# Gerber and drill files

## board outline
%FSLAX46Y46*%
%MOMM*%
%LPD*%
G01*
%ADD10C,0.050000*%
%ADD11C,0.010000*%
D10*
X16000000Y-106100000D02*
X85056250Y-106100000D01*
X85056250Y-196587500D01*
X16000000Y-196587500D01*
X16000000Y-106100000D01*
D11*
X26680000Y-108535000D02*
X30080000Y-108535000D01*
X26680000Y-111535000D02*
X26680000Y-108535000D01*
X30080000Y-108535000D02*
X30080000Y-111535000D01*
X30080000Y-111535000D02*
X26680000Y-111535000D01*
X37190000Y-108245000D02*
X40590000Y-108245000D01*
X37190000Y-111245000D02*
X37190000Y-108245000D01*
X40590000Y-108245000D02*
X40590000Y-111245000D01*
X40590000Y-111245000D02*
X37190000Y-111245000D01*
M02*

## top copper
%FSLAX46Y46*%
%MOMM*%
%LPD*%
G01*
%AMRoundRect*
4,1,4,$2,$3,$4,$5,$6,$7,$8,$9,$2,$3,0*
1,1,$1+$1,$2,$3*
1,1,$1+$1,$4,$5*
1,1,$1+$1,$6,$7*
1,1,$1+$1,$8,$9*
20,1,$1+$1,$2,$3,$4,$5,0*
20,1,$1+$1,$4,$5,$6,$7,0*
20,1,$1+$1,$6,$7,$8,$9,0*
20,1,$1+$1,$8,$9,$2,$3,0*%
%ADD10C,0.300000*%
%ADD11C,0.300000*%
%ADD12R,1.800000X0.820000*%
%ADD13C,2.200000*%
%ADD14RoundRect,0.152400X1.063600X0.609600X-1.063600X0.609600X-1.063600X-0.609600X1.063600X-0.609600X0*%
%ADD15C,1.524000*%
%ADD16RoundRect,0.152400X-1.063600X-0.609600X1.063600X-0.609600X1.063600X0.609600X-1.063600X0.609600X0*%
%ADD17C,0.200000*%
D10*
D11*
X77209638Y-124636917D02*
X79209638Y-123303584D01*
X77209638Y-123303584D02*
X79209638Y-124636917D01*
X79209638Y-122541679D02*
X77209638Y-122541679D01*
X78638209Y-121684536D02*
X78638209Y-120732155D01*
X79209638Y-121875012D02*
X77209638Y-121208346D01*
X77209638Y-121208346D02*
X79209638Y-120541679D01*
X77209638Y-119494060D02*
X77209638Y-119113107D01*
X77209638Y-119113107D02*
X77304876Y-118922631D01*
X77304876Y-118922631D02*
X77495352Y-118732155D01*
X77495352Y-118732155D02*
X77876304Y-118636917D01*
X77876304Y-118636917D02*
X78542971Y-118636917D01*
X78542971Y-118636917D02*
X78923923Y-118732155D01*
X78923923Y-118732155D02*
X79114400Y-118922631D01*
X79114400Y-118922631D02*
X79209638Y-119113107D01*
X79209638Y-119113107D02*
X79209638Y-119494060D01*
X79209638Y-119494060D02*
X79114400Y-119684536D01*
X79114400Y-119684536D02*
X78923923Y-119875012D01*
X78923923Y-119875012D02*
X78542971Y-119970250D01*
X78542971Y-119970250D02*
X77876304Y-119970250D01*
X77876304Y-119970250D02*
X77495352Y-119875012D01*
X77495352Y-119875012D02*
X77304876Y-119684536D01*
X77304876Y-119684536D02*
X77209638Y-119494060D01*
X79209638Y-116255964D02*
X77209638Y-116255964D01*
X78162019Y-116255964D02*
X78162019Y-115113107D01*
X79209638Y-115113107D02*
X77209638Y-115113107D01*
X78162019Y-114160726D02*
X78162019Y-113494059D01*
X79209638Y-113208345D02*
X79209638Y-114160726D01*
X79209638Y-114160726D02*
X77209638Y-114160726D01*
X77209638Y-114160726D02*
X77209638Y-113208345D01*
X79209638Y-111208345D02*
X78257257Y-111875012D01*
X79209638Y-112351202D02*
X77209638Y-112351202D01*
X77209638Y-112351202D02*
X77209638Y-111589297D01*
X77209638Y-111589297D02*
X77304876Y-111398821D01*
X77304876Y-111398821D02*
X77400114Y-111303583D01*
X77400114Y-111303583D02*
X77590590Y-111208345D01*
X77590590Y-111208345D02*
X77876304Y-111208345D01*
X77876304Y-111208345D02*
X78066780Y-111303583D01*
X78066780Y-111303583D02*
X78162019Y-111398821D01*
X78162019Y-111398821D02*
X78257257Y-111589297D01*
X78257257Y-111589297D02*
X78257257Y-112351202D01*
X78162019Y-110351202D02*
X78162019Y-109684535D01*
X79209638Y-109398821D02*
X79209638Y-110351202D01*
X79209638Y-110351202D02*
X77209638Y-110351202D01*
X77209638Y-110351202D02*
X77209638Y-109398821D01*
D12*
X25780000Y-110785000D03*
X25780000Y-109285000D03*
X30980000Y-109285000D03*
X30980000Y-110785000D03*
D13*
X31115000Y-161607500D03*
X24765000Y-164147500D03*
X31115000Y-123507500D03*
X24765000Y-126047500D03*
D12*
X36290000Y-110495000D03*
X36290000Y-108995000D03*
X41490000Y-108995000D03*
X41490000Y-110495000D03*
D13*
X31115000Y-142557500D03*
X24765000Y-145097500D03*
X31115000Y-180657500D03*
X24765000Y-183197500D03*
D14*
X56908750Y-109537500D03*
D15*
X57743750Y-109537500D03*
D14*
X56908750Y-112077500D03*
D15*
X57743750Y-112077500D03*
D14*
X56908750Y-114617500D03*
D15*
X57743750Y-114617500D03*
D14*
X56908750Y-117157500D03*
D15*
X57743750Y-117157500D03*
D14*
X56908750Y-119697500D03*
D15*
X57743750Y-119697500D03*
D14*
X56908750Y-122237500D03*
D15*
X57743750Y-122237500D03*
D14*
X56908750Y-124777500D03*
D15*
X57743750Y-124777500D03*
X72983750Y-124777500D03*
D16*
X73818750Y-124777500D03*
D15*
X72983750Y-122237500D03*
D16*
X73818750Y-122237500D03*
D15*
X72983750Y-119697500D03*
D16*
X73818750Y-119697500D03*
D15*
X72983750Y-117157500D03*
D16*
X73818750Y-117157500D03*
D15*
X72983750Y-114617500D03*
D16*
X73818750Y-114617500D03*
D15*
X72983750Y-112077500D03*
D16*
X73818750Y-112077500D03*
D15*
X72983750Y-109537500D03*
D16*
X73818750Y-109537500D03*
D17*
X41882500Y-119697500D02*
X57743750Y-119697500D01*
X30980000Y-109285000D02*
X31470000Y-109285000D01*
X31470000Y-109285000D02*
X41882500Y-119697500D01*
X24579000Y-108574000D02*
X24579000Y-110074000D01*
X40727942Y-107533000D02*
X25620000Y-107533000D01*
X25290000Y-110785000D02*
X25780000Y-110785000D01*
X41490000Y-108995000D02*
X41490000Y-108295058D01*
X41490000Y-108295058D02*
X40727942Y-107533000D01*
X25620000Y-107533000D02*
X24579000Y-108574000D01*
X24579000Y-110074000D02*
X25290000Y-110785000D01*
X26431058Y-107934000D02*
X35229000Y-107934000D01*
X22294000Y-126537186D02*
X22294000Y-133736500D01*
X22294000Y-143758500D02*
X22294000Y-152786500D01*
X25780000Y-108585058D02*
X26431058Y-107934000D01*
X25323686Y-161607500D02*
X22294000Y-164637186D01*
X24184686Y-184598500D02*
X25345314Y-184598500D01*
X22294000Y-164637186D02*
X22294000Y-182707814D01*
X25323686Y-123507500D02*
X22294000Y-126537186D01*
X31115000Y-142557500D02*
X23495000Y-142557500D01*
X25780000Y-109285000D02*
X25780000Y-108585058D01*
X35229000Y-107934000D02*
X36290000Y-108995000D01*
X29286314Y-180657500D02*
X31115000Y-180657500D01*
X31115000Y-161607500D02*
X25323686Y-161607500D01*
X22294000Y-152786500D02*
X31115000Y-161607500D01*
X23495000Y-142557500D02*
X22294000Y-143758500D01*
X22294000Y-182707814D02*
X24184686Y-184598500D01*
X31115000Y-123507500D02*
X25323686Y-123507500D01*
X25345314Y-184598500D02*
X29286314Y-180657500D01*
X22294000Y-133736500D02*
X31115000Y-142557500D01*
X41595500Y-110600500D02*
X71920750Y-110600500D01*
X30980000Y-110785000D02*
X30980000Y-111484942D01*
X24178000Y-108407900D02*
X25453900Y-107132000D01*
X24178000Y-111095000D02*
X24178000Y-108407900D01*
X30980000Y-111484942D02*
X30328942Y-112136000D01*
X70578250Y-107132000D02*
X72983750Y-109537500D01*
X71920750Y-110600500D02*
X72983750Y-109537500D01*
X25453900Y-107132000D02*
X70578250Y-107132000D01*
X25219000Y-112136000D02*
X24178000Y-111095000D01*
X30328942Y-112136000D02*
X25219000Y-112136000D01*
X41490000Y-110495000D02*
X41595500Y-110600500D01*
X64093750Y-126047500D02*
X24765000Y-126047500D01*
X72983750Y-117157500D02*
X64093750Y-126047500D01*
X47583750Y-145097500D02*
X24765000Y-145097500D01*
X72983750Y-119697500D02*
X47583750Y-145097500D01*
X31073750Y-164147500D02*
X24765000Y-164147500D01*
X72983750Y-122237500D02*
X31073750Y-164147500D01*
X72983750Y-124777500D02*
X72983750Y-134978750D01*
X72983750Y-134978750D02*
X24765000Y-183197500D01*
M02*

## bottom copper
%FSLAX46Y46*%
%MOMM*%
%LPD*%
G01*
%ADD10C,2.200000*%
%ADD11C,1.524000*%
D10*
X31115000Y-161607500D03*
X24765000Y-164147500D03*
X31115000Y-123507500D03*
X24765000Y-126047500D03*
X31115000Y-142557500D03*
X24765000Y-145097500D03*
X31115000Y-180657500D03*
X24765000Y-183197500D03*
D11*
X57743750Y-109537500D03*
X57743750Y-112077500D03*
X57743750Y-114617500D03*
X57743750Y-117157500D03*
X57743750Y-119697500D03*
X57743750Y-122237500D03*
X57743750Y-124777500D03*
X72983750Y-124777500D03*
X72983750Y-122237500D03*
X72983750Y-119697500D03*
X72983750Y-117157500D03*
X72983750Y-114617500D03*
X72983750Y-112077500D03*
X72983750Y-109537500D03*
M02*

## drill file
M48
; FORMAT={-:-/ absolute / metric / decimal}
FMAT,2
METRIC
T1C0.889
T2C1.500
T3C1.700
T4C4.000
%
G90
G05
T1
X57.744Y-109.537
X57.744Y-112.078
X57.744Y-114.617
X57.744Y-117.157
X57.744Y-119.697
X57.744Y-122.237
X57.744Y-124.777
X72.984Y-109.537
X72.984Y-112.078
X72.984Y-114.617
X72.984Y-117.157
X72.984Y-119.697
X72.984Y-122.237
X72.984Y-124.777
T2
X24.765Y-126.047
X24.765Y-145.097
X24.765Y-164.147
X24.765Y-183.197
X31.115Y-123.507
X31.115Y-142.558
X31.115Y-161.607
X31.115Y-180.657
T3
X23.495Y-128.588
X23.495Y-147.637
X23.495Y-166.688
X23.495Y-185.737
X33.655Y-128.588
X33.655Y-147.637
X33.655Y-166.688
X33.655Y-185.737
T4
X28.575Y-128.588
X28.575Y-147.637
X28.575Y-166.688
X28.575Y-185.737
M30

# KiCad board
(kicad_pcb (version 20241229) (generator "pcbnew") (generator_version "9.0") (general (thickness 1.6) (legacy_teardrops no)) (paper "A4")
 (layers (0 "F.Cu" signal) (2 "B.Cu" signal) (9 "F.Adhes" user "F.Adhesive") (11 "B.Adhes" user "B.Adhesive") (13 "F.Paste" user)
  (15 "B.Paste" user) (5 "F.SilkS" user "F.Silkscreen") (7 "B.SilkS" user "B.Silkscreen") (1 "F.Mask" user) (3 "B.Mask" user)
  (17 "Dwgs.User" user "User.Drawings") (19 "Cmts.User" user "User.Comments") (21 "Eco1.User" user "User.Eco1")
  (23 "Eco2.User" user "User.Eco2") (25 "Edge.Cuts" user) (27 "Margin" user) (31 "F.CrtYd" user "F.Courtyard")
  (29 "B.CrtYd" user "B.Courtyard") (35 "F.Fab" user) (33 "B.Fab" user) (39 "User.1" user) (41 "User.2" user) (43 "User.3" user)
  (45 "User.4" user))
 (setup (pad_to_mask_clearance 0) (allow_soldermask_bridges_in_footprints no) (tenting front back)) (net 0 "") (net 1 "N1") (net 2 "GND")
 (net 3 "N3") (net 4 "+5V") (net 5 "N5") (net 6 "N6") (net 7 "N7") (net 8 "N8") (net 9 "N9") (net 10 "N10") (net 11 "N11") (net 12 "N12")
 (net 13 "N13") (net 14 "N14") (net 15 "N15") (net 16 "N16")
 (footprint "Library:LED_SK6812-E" (layer "F.Cu") (at 28.38 110.035 180)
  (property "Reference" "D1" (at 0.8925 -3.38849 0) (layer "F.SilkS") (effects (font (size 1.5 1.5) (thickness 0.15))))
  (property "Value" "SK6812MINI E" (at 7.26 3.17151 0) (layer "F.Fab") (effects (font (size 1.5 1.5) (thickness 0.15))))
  (fp_line (start 1.7 1.5) (end -1.7 1.5) (stroke (width 0.01) (type solid)) (layer "Edge.Cuts"))
  (fp_line (start 1.7 -1.5) (end 1.7 1.5) (stroke (width 0.01) (type solid)) (layer "Edge.Cuts"))
  (fp_line (start -1.7 1.5) (end -1.7 -1.5) (stroke (width 0.01) (type solid)) (layer "Edge.Cuts"))
  (fp_line (start -1.7 -1.5) (end 1.7 -1.5) (stroke (width 0.01) (type solid)) (layer "Edge.Cuts"))
  (pad "1" smd rect (at 2.6 -0.75 180) (size 1.8 0.82) (layers "F.Cu" "F.Mask" "F.Paste") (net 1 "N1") (solder_mask_margin 0.102))
  (pad "2" smd rect (at 2.6 0.75 180) (size 1.8 0.82) (layers "F.Cu" "F.Mask" "F.Paste") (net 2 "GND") (solder_mask_margin 0.102))
  (pad "3" smd rect (at -2.6 0.75 180) (size 1.8 0.82) (layers "F.Cu" "F.Mask" "F.Paste") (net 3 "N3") (solder_mask_margin 0.102))
  (pad "4" smd rect (at -2.6 -0.75 180) (size 1.8 0.82) (layers "F.Cu" "F.Mask" "F.Paste") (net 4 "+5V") (solder_mask_margin 0.102)))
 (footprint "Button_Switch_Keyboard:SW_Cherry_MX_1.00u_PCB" (layer "F.Cu") (at 31.115 161.6075)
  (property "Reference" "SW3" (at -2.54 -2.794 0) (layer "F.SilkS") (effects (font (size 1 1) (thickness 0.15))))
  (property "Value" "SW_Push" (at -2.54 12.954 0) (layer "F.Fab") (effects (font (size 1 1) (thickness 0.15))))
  (pad "" np_thru_hole circle (at -7.62 5.08) (size 1.7 1.7) (drill 1.7) (layers "*.Cu" "*.Mask"))
  (pad "" np_thru_hole circle (at -2.54 5.08) (size 4 4) (drill 4) (layers "*.Cu" "*.Mask"))
  (pad "" np_thru_hole circle (at 2.54 5.08) (size 1.7 1.7) (drill 1.7) (layers "*.Cu" "*.Mask"))
  (pad "1" thru_hole circle (at 0 0) (size 2.2 2.2) (drill 1.5) (layers "*.Cu" "*.Mask") (remove_unused_layers no) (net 2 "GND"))
  (pad "2" thru_hole circle (at -6.35 2.54) (size 2.2 2.2) (drill 1.5) (layers "*.Cu" "*.Mask") (remove_unused_layers no) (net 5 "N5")))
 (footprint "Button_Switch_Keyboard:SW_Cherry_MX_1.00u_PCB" (layer "F.Cu") (at 31.115 123.5075)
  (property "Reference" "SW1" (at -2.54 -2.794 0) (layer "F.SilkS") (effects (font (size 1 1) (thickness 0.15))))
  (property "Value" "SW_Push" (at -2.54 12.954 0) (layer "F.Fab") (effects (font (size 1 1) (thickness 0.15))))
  (pad "" np_thru_hole circle (at -7.62 5.08) (size 1.7 1.7) (drill 1.7) (layers "*.Cu" "*.Mask"))
  (pad "" np_thru_hole circle (at -2.54 5.08) (size 4 4) (drill 4) (layers "*.Cu" "*.Mask"))
  (pad "" np_thru_hole circle (at 2.54 5.08) (size 1.7 1.7) (drill 1.7) (layers "*.Cu" "*.Mask"))
  (pad "1" thru_hole circle (at 0 0) (size 2.2 2.2) (drill 1.5) (layers "*.Cu" "*.Mask") (remove_unused_layers no) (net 2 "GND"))
  (pad "2" thru_hole circle (at -6.35 2.54) (size 2.2 2.2) (drill 1.5) (layers "*.Cu" "*.Mask") (remove_unused_layers no) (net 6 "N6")))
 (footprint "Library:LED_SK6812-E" (layer "F.Cu") (at 38.89 109.745 180)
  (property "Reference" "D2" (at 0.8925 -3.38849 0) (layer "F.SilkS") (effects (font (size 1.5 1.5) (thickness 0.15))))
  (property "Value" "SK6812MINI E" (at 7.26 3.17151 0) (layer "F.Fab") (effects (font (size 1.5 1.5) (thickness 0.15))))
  (fp_line (start 1.7 1.5) (end -1.7 1.5) (stroke (width 0.01) (type solid)) (layer "Edge.Cuts"))
  (fp_line (start 1.7 -1.5) (end 1.7 1.5) (stroke (width 0.01) (type solid)) (layer "Edge.Cuts"))
  (fp_line (start -1.7 1.5) (end -1.7 -1.5) (stroke (width 0.01) (type solid)) (layer "Edge.Cuts"))
  (fp_line (start -1.7 -1.5) (end 1.7 -1.5) (stroke (width 0.01) (type solid)) (layer "Edge.Cuts"))
  (pad "1" smd rect (at 2.6 -0.75 180) (size 1.8 0.82) (layers "F.Cu" "F.Mask" "F.Paste") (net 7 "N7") (solder_mask_margin 0.102))
  (pad "2" smd rect (at 2.6 0.75 180) (size 1.8 0.82) (layers "F.Cu" "F.Mask" "F.Paste") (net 2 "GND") (solder_mask_margin 0.102))
  (pad "3" smd rect (at -2.6 0.75 180) (size 1.8 0.82) (layers "F.Cu" "F.Mask" "F.Paste") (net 1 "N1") (solder_mask_margin 0.102))
  (pad "4" smd rect (at -2.6 -0.75 180) (size 1.8 0.82) (layers "F.Cu" "F.Mask" "F.Paste") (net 4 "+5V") (solder_mask_margin 0.102)))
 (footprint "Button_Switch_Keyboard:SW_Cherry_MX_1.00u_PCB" (layer "F.Cu") (at 31.115 142.5575)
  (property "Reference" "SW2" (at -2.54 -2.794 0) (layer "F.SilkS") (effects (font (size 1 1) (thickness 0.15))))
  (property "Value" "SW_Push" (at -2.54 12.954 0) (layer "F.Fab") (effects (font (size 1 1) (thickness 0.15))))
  (pad "" np_thru_hole circle (at -7.62 5.08) (size 1.7 1.7) (drill 1.7) (layers "*.Cu" "*.Mask"))
  (pad "" np_thru_hole circle (at -2.54 5.08) (size 4 4) (drill 4) (layers "*.Cu" "*.Mask"))
  (pad "" np_thru_hole circle (at 2.54 5.08) (size 1.7 1.7) (drill 1.7) (layers "*.Cu" "*.Mask"))
  (pad "1" thru_hole circle (at 0 0) (size 2.2 2.2) (drill 1.5) (layers "*.Cu" "*.Mask") (remove_unused_layers no) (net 2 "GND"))
  (pad "2" thru_hole circle (at -6.35 2.54) (size 2.2 2.2) (drill 1.5) (layers "*.Cu" "*.Mask") (remove_unused_layers no) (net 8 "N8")))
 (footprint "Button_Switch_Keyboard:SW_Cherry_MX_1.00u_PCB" (layer "F.Cu") (at 31.115 180.6575)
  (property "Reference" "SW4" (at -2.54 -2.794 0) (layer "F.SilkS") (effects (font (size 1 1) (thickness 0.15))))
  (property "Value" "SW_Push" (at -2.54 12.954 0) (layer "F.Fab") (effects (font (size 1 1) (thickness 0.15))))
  (pad "" np_thru_hole circle (at -7.62 5.08) (size 1.7 1.7) (drill 1.7) (layers "*.Cu" "*.Mask"))
  (pad "" np_thru_hole circle (at -2.54 5.08) (size 4 4) (drill 4) (layers "*.Cu" "*.Mask"))
  (pad "" np_thru_hole circle (at 2.54 5.08) (size 1.7 1.7) (drill 1.7) (layers "*.Cu" "*.Mask"))
  (pad "1" thru_hole circle (at 0 0) (size 2.2 2.2) (drill 1.5) (layers "*.Cu" "*.Mask") (remove_unused_layers no) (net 2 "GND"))
  (pad "2" thru_hole circle (at -6.35 2.54) (size 2.2 2.2) (drill 1.5) (layers "*.Cu" "*.Mask") (remove_unused_layers no) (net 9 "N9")))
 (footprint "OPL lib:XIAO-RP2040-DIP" (layer "F.Cu") (at 65.36375 117.1575)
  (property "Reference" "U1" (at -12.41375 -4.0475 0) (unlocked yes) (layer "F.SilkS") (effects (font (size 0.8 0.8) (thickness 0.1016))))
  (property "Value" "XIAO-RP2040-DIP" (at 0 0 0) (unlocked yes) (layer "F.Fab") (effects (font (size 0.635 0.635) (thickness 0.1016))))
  (pad "1" smd roundrect (at -8.455 -7.62 180) (size 2.432 1.524) (layers "F.Cu" "F.Mask") (roundrect_rratio 0.1) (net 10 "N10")
   (thermal_bridge_angle 45))
  (pad "1" thru_hole circle (at -7.62 -7.62 180) (size 1.524 1.524) (drill 0.889) (layers "*.Cu" "*.Mask") (remove_unused_layers no)
   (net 10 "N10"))
  (pad "2" smd roundrect (at -8.455 -5.08 180) (size 2.432 1.524) (layers "F.Cu" "F.Mask") (roundrect_rratio 0.1) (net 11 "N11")
   (thermal_bridge_angle 45))
  (pad "2" thru_hole circle (at -7.62 -5.08 180) (size 1.524 1.524) (drill 0.889) (layers "*.Cu" "*.Mask") (remove_unused_layers no)
   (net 11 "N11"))
  (pad "3" smd roundrect (at -8.455 -2.54 180) (size 2.432 1.524) (layers "F.Cu" "F.Mask") (roundrect_rratio 0.1) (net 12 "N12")
   (thermal_bridge_angle 45))
  (pad "3" thru_hole circle (at -7.62 -2.54 180) (size 1.524 1.524) (drill 0.889) (layers "*.Cu" "*.Mask") (remove_unused_layers no)
   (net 12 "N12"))
  (pad "4" smd roundrect (at -8.455 0 180) (size 2.432 1.524) (layers "F.Cu" "F.Mask") (roundrect_rratio 0.1) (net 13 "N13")
   (thermal_bridge_angle 45))
  (pad "4" thru_hole circle (at -7.62 0 180) (size 1.524 1.524) (drill 0.889) (layers "*.Cu" "*.Mask") (remove_unused_layers no)
   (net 13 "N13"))
  (pad "5" smd roundrect (at -8.455 2.54 180) (size 2.432 1.524) (layers "F.Cu" "F.Mask") (roundrect_rratio 0.1) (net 3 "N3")
   (thermal_bridge_angle 45))
  (pad "5" thru_hole circle (at -7.62 2.54 180) (size 1.524 1.524) (drill 0.889) (layers "*.Cu" "*.Mask") (remove_unused_layers no)
   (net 3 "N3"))
  (pad "6" smd roundrect (at -8.455 5.08 180) (size 2.432 1.524) (layers "F.Cu" "F.Mask") (roundrect_rratio 0.1) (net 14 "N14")
   (thermal_bridge_angle 45))
  (pad "6" thru_hole circle (at -7.62 5.08 180) (size 1.524 1.524) (drill 0.889) (layers "*.Cu" "*.Mask") (remove_unused_layers no)
   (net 14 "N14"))
  (pad "7" smd roundrect (at -8.455 7.62 180) (size 2.432 1.524) (layers "F.Cu" "F.Mask") (roundrect_rratio 0.1) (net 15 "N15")
   (thermal_bridge_angle 45))
  (pad "7" thru_hole circle (at -7.62 7.62 180) (size 1.524 1.524) (drill 0.889) (layers "*.Cu" "*.Mask") (remove_unused_layers no)
   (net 15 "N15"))
  (pad "8" thru_hole circle (at 7.62 7.62) (size 1.524 1.524) (drill 0.889) (layers "*.Cu" "*.Mask") (remove_unused_layers no) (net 9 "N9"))
  (pad "8" smd roundrect (at 8.455 7.62) (size 2.432 1.524) (layers "F.Cu" "F.Mask") (roundrect_rratio 0.1) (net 9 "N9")
   (thermal_bridge_angle 45))
  (pad "9" thru_hole circle (at 7.62 5.08) (size 1.524 1.524) (drill 0.889) (layers "*.Cu" "*.Mask") (remove_unused_layers no) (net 5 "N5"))
  (pad "9" smd roundrect (at 8.455 5.08) (size 2.432 1.524) (layers "F.Cu" "F.Mask") (roundrect_rratio 0.1) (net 5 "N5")
   (thermal_bridge_angle 45))
  (pad "10" thru_hole circle (at 7.62 2.54) (size 1.524 1.524) (drill 0.889) (layers "*.Cu" "*.Mask") (remove_unused_layers no) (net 8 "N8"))
  (pad "10" smd roundrect (at 8.455 2.54) (size 2.432 1.524) (layers "F.Cu" "F.Mask") (roundrect_rratio 0.1) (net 8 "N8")
   (thermal_bridge_angle 45))
  (pad "11" thru_hole circle (at 7.62 0) (size 1.524 1.524) (drill 0.889) (layers "*.Cu" "*.Mask") (remove_unused_layers no) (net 6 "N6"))
  (pad "11" smd roundrect (at 8.455 0) (size 2.432 1.524) (layers "F.Cu" "F.Mask") (roundrect_rratio 0.1) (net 6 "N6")
   (thermal_bridge_angle 45))
  (pad "12" thru_hole circle (at 7.62 -2.54) (size 1.524 1.524) (drill 0.889) (layers "*.Cu" "*.Mask") (remove_unused_layers no)
   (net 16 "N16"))
  (pad "12" smd roundrect (at 8.455 -2.54) (size 2.432 1.524) (layers "F.Cu" "F.Mask") (roundrect_rratio 0.1) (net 16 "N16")
   (thermal_bridge_angle 45))
  (pad "13" thru_hole circle (at 7.62 -5.08) (size 1.524 1.524) (drill 0.889) (layers "*.Cu" "*.Mask") (remove_unused_layers no)
   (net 2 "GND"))
  (pad "13" smd roundrect (at 8.455 -5.08) (size 2.432 1.524) (layers "F.Cu" "F.Mask") (roundrect_rratio 0.1) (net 2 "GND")
   (thermal_bridge_angle 45))
  (pad "14" thru_hole circle (at 7.62 -7.62) (size 1.524 1.524) (drill 0.889) (layers "*.Cu" "*.Mask") (remove_unused_layers no)
   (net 4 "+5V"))
  (pad "14" smd roundrect (at 8.455 -7.62) (size 2.432 1.524) (layers "F.Cu" "F.Mask") (roundrect_rratio 0.1) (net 4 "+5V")
   (thermal_bridge_angle 45)))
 (gr_rect (start 16 106.1) (end 85.05625 196.5875) (stroke (width 0.05) (type default)) (fill no) (layer "Edge.Cuts"))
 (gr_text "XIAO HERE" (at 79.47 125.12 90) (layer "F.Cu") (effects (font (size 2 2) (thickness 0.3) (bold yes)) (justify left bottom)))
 (segment (start 41.8825 119.6975) (end 57.74375 119.6975) (width 0.2) (layer "F.Cu") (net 3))
 (segment (start 30.98 109.285) (end 31.47 109.285) (width 0.2) (layer "F.Cu") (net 3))
 (segment (start 31.47 109.285) (end 41.8825 119.6975) (width 0.2) (layer "F.Cu") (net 3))
 (segment (start 24.579 108.574) (end 24.579 110.074) (width 0.2) (layer "F.Cu") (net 1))
 (segment (start 40.727942 107.533) (end 25.62 107.533) (width 0.2) (layer "F.Cu") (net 1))
 (segment (start 25.29 110.785) (end 25.78 110.785) (width 0.2) (layer "F.Cu") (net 1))
 (segment (start 41.49 108.995) (end 41.49 108.295058) (width 0.2) (layer "F.Cu") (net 1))
 (segment (start 41.49 108.295058) (end 40.727942 107.533) (width 0.2) (layer "F.Cu") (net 1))
 (segment (start 25.62 107.533) (end 24.579 108.574) (width 0.2) (layer "F.Cu") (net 1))
 (segment (start 24.579 110.074) (end 25.29 110.785) (width 0.2) (layer "F.Cu") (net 1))
 (segment (start 26.431058 107.934) (end 35.229 107.934) (width 0.2) (layer "F.Cu") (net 2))
 (segment (start 22.294 126.537186) (end 22.294 133.7365) (width 0.2) (layer "F.Cu") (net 2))
 (segment (start 22.294 143.7585) (end 22.294 152.7865) (width 0.2) (layer "F.Cu") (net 2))
 (segment (start 25.78 108.585058) (end 26.431058 107.934) (width 0.2) (layer "F.Cu") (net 2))
 (segment (start 25.323686 161.6075) (end 22.294 164.637186) (width 0.2) (layer "F.Cu") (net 2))
 (segment (start 24.184686 184.5985) (end 25.345314 184.5985) (width 0.2) (layer "F.Cu") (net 2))
 (segment (start 22.294 164.637186) (end 22.294 182.707814) (width 0.2) (layer "F.Cu") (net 2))
 (segment (start 25.323686 123.5075) (end 22.294 126.537186) (width 0.2) (layer "F.Cu") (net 2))
 (segment (start 31.115 142.5575) (end 23.495 142.5575) (width 0.2) (layer "F.Cu") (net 2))
 (segment (start 25.78 109.285) (end 25.78 108.585058) (width 0.2) (layer "F.Cu") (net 2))
 (segment (start 35.229 107.934) (end 36.29 108.995) (width 0.2) (layer "F.Cu") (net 2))
 (segment (start 29.286314 180.6575) (end 31.115 180.6575) (width 0.2) (layer "F.Cu") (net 2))
 (segment (start 31.115 161.6075) (end 25.323686 161.6075) (width 0.2) (layer "F.Cu") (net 2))
 (segment (start 22.294 152.7865) (end 31.115 161.6075) (width 0.2) (layer "F.Cu") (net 2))
 (segment (start 23.495 142.5575) (end 22.294 143.7585) (width 0.2) (layer "F.Cu") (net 2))
 (segment (start 22.294 182.707814) (end 24.184686 184.5985) (width 0.2) (layer "F.Cu") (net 2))
 (segment (start 31.115 123.5075) (end 25.323686 123.5075) (width 0.2) (layer "F.Cu") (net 2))
 (segment (start 25.345314 184.5985) (end 29.286314 180.6575) (width 0.2) (layer "F.Cu") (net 2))
 (segment (start 22.294 133.7365) (end 31.115 142.5575) (width 0.2) (layer "F.Cu") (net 2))
 (segment (start 41.5955 110.6005) (end 71.92075 110.6005) (width 0.2) (layer "F.Cu") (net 4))
 (segment (start 30.98 110.785) (end 30.98 111.484942) (width 0.2) (layer "F.Cu") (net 4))
 (segment (start 24.178 108.4079) (end 25.4539 107.132) (width 0.2) (layer "F.Cu") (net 4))
 (segment (start 24.178 111.095) (end 24.178 108.4079) (width 0.2) (layer "F.Cu") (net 4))
 (segment (start 30.98 111.484942) (end 30.328942 112.136) (width 0.2) (layer "F.Cu") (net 4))
 (segment (start 70.57825 107.132) (end 72.98375 109.5375) (width 0.2) (layer "F.Cu") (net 4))
 (segment (start 71.92075 110.6005) (end 72.98375 109.5375) (width 0.2) (layer "F.Cu") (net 4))
 (segment (start 25.4539 107.132) (end 70.57825 107.132) (width 0.2) (layer "F.Cu") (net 4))
 (segment (start 25.219 112.136) (end 24.178 111.095) (width 0.2) (layer "F.Cu") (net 4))
 (segment (start 30.328942 112.136) (end 25.219 112.136) (width 0.2) (layer "F.Cu") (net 4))
 (segment (start 41.49 110.495) (end 41.5955 110.6005) (width 0.2) (layer "F.Cu") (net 4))
 (segment (start 64.09375 126.0475) (end 24.765 126.0475) (width 0.2) (layer "F.Cu") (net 6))
 (segment (start 72.98375 117.1575) (end 64.09375 126.0475) (width 0.2) (layer "F.Cu") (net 6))
 (segment (start 47.58375 145.0975) (end 24.765 145.0975) (width 0.2) (layer "F.Cu") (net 8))
 (segment (start 72.98375 119.6975) (end 47.58375 145.0975) (width 0.2) (layer "F.Cu") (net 8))
 (segment (start 31.07375 164.1475) (end 24.765 164.1475) (width 0.2) (layer "F.Cu") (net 5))
 (segment (start 72.98375 122.2375) (end 31.07375 164.1475) (width 0.2) (layer "F.Cu") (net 5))
 (segment (start 72.98375 124.7775) (end 72.98375 134.97875) (width 0.2) (layer "F.Cu") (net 9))
 (segment (start 72.98375 134.97875) (end 24.765 183.1975) (width 0.2) (layer "F.Cu") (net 9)))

